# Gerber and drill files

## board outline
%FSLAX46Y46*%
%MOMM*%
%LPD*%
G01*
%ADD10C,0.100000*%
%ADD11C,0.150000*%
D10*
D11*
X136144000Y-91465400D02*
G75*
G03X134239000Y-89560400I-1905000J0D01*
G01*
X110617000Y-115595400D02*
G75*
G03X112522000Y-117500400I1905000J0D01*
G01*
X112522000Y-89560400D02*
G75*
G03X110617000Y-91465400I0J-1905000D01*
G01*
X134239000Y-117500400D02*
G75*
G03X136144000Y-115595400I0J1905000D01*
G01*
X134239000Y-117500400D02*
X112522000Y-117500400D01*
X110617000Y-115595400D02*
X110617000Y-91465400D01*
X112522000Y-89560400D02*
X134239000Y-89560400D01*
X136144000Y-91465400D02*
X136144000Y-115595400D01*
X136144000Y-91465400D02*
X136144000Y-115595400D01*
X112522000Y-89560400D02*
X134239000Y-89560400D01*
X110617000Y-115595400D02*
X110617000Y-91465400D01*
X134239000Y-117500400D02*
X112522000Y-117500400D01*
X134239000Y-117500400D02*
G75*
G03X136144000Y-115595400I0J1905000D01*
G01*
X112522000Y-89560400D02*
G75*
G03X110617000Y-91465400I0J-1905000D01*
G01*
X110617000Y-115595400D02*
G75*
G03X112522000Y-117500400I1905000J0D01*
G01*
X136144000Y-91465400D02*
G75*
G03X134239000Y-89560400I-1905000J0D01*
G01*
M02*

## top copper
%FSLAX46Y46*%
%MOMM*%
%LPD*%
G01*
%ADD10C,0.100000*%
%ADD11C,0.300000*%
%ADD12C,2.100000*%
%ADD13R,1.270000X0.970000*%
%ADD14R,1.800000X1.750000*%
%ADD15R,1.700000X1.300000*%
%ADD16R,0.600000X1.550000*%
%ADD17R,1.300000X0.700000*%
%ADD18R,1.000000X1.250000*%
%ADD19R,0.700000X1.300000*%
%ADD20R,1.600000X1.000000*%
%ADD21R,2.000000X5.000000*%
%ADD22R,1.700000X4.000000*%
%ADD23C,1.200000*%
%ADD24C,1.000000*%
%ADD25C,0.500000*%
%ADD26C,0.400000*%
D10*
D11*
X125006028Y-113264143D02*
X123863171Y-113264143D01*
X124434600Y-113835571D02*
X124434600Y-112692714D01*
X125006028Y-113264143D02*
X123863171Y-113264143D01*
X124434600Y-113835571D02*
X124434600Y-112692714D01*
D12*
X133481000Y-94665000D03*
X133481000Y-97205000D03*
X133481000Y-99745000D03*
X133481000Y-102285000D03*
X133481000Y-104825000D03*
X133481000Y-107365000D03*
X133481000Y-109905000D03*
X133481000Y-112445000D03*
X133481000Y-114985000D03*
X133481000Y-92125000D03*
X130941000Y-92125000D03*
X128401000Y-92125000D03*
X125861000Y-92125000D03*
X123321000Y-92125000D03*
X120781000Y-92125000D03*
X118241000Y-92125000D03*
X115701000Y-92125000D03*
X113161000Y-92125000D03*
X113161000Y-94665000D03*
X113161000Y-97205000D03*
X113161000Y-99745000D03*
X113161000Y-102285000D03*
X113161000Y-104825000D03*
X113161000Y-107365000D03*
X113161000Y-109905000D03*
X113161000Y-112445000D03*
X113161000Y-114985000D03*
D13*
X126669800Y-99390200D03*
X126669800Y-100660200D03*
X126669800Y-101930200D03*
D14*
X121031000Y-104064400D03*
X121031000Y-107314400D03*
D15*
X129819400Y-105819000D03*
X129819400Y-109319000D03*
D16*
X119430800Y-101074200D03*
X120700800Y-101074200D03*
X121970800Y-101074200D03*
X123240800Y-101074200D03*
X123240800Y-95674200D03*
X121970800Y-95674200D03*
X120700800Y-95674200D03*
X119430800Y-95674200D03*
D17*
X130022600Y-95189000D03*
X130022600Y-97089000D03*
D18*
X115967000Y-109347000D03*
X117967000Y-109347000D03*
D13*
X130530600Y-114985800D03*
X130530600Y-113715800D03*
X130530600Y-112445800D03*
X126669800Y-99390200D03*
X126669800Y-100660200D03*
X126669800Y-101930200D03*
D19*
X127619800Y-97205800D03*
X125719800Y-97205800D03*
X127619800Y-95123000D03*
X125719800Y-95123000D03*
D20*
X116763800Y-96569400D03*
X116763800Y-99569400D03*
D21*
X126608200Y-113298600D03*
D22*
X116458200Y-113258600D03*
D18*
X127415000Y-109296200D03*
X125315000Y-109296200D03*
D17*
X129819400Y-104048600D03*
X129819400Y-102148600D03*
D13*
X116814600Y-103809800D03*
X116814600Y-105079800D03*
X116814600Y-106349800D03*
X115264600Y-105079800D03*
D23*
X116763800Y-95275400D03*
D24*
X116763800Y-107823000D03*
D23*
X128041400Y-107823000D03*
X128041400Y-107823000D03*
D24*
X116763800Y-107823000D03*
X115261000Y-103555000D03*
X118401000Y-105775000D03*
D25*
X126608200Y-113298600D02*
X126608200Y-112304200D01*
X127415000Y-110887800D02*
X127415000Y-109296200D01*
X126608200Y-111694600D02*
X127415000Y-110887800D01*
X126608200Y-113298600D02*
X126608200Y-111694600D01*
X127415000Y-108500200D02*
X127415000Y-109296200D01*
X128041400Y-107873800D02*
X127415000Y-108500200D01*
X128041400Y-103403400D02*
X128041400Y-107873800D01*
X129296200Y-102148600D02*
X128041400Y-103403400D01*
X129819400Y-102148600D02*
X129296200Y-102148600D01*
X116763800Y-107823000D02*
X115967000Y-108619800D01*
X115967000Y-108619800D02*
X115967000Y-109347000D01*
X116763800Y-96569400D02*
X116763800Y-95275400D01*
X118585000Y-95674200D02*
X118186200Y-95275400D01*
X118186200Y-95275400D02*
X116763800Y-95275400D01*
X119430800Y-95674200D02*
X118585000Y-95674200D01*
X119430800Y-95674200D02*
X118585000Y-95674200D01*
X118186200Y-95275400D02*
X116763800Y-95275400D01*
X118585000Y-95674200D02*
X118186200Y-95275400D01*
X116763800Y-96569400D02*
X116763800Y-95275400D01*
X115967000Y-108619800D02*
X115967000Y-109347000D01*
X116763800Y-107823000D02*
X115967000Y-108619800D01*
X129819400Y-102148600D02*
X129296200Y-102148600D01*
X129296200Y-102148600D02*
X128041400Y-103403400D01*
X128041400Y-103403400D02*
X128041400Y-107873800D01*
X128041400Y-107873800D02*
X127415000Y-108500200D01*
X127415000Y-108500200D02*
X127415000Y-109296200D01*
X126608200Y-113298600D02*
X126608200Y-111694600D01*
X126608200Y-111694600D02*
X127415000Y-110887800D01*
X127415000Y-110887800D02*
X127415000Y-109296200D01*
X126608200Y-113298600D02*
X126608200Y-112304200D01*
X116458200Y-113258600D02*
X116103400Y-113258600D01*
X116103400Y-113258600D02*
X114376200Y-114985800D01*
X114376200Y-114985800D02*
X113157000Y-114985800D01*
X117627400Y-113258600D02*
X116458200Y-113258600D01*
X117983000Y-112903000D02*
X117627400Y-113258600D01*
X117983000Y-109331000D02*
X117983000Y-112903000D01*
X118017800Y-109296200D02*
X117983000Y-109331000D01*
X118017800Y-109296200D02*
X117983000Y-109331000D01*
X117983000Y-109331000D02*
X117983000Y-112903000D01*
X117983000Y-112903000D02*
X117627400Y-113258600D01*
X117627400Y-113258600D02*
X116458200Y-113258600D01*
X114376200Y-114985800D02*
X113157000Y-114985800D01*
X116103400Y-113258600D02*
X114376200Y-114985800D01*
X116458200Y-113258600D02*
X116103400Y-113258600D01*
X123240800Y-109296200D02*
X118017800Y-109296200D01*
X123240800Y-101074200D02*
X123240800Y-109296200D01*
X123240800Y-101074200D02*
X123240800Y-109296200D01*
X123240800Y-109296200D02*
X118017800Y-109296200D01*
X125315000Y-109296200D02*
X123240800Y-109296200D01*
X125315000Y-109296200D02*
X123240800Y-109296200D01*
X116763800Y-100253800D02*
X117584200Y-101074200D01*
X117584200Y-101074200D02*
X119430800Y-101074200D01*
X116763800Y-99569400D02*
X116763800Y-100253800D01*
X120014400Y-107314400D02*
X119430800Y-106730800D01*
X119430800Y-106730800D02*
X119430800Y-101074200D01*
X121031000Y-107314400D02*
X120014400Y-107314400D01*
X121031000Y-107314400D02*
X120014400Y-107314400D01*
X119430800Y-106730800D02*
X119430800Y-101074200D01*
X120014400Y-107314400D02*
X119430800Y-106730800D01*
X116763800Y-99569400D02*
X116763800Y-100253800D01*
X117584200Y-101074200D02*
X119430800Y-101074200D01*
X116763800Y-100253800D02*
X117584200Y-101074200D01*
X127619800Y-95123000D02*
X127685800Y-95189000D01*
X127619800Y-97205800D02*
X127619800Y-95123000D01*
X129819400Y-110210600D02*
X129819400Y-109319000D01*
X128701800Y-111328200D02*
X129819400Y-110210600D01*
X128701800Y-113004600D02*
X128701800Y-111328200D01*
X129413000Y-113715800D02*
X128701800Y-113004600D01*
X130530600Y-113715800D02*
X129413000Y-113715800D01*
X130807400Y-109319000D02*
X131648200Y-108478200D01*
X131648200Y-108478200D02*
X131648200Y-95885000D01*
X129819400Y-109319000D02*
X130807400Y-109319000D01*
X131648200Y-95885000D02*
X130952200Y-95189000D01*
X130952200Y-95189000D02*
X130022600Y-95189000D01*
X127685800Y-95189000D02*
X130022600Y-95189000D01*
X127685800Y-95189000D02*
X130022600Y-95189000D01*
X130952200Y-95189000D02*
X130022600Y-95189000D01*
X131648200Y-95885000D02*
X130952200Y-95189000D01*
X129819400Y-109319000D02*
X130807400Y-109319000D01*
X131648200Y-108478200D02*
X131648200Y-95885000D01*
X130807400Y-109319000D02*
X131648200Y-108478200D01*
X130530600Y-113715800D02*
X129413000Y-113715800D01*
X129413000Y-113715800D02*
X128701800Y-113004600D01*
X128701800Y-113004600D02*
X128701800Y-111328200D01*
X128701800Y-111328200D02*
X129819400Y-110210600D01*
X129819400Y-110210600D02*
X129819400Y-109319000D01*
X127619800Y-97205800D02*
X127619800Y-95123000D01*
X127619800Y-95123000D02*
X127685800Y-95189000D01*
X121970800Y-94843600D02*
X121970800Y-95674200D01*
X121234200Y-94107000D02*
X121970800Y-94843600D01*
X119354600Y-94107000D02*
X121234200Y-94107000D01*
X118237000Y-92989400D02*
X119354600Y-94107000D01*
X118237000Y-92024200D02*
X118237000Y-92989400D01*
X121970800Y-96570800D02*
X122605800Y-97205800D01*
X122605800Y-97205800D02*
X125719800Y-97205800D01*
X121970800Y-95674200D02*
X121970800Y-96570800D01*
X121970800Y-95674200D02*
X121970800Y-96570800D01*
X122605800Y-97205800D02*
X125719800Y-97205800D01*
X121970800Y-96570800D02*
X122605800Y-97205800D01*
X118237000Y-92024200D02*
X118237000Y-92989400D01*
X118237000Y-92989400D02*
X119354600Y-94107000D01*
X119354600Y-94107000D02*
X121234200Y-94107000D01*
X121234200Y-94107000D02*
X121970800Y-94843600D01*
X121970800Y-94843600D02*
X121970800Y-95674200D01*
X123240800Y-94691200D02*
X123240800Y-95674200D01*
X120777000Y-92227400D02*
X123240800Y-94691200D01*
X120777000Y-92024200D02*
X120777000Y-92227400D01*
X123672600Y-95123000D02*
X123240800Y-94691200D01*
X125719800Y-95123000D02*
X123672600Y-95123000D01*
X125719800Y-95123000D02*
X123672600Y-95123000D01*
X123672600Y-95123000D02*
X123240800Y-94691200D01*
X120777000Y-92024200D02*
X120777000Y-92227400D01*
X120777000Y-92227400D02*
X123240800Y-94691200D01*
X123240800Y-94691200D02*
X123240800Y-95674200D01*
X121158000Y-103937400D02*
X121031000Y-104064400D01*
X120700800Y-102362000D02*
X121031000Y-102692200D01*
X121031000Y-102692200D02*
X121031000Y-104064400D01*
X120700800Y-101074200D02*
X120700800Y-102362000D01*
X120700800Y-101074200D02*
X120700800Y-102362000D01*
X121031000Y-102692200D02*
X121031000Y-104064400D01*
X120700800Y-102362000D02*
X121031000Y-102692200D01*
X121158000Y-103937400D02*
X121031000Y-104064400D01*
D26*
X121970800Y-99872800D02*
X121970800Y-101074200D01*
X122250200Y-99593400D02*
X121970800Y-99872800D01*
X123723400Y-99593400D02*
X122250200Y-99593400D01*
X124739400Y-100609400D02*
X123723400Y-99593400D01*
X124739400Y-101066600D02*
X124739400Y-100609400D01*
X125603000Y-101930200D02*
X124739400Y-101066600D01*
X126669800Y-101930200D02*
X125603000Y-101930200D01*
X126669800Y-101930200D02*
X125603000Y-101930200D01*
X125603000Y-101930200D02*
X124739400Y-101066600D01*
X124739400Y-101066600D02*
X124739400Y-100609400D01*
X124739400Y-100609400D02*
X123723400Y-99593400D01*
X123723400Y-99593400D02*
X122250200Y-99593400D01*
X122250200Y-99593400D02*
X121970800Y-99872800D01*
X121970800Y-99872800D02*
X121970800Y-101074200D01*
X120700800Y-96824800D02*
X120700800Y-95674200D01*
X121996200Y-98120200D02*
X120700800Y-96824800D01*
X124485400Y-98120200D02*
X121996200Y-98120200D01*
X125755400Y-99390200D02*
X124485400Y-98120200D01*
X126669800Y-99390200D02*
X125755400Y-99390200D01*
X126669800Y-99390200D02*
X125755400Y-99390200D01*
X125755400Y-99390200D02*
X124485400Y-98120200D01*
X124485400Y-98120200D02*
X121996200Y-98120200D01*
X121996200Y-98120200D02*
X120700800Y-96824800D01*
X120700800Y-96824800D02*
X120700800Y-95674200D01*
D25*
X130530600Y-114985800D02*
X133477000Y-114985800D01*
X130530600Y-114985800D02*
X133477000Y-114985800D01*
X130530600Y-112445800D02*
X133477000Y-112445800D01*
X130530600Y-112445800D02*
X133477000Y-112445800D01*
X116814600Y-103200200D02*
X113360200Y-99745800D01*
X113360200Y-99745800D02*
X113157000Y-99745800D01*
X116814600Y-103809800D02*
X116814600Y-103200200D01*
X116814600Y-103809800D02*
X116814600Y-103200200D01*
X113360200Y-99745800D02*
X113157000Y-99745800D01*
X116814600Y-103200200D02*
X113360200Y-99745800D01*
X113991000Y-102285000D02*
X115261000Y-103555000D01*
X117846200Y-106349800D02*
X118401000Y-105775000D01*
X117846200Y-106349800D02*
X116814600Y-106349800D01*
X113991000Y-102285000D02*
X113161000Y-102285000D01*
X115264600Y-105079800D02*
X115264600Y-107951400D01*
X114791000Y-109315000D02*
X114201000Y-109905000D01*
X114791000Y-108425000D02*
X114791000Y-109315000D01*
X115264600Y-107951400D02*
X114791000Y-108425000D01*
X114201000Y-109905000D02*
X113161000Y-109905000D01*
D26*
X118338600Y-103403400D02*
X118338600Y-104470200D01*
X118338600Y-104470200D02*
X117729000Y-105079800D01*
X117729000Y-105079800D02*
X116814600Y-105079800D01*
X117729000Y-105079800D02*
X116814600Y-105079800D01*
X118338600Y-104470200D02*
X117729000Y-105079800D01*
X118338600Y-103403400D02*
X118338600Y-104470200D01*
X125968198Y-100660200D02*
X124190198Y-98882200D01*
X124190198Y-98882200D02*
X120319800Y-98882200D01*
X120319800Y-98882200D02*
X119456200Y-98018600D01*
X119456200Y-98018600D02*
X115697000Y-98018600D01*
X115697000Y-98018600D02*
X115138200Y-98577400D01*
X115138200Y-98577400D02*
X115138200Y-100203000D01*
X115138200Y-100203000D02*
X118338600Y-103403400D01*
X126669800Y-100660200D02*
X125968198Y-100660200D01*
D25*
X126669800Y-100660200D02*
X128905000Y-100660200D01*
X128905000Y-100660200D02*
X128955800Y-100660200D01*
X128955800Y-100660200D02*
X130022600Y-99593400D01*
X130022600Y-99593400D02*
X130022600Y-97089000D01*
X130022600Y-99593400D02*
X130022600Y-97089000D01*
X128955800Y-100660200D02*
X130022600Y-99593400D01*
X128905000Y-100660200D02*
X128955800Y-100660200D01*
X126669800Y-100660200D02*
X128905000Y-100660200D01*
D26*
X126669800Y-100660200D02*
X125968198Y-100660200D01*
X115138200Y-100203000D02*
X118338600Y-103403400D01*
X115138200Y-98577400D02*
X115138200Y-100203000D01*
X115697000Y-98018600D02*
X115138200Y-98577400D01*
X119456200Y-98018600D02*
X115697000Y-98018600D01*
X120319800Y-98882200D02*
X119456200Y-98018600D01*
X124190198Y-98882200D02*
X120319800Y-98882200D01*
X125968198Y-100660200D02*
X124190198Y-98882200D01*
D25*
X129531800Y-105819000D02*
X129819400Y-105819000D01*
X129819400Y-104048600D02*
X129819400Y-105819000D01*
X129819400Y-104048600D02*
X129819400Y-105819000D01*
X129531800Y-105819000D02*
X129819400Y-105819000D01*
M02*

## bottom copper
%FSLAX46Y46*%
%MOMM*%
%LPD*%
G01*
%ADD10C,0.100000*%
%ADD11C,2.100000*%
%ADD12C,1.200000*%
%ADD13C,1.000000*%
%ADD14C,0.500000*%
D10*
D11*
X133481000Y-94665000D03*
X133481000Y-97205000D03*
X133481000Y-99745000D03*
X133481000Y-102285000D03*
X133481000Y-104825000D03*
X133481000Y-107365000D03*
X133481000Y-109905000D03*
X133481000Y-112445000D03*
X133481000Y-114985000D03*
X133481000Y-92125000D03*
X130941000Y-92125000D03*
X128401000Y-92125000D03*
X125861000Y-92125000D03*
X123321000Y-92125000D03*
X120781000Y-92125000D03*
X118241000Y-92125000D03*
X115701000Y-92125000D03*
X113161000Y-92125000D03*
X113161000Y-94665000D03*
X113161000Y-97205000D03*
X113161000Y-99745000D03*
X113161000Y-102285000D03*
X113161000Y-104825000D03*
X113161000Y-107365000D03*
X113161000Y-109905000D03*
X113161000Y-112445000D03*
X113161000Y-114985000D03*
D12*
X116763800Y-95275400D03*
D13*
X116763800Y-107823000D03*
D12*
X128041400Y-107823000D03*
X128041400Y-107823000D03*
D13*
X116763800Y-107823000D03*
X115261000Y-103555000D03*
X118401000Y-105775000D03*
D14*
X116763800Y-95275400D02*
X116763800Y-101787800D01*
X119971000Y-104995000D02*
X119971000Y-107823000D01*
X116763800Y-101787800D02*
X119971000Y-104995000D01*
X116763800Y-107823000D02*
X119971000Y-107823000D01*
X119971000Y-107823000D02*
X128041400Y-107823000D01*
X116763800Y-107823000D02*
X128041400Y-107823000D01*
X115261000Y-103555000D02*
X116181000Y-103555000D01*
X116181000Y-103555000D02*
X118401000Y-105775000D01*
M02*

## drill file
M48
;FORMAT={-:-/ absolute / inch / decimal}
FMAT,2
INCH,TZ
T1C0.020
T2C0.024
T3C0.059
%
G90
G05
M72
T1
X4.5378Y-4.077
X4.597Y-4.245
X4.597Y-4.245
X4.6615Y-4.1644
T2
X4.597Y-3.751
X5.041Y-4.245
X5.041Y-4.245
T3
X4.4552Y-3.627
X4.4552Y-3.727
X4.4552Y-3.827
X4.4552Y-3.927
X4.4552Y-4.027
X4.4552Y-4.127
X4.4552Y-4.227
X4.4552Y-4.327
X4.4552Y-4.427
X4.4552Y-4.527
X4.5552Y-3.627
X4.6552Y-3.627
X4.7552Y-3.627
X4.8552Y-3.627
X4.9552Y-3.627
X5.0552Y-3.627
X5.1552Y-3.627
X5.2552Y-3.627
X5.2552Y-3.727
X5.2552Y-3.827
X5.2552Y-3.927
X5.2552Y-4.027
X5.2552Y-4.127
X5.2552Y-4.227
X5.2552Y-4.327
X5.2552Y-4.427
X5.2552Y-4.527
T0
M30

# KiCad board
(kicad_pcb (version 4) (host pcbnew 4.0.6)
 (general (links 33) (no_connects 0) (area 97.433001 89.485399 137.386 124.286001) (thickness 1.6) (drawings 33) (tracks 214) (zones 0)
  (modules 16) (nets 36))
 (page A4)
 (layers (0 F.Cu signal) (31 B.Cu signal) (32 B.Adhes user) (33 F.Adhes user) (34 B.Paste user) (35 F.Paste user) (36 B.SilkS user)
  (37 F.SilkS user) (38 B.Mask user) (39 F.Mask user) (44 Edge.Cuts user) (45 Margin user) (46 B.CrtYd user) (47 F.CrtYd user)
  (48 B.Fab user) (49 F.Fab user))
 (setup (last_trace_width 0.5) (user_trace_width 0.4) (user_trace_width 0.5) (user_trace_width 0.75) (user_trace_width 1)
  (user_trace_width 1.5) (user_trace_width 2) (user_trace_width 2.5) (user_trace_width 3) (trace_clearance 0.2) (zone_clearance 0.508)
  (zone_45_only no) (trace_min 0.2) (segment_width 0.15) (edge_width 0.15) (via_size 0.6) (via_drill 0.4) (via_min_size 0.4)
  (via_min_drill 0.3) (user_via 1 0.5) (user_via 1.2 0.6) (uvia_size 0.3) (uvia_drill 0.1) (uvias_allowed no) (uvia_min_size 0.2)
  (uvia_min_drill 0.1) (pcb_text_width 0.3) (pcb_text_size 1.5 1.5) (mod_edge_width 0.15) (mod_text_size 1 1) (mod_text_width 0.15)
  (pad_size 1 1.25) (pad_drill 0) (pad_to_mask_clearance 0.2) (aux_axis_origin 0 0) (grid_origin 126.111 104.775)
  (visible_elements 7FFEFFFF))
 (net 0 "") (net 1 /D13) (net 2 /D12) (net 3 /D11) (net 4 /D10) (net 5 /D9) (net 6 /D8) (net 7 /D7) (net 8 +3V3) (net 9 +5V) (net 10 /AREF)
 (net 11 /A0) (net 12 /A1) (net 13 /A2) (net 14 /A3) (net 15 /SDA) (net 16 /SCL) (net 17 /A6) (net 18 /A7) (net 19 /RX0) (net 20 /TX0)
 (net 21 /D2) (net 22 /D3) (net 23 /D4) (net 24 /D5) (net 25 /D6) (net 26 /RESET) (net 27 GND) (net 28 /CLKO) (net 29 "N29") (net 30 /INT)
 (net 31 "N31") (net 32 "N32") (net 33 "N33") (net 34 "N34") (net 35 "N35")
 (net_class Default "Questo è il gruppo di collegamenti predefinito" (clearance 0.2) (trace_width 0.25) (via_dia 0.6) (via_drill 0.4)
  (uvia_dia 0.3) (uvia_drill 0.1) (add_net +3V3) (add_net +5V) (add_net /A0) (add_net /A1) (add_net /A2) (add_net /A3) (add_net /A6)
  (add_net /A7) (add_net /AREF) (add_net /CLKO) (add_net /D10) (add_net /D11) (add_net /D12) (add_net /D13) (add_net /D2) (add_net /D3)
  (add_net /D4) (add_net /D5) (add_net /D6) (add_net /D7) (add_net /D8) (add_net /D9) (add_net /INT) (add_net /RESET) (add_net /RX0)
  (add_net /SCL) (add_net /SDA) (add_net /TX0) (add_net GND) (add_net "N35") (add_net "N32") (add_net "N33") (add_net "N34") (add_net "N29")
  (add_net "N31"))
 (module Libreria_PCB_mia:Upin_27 (layer B.Cu) (at 133.481 114.985 180)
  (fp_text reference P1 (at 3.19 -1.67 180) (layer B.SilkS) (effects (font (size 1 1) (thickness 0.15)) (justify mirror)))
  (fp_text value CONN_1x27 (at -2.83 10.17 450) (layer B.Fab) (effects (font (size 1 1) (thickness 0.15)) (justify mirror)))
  (pad 9 thru_hole circle (at 0 20.32 180) (size 2.1 2.1) (drill 1.5) (layers *.Cu *.Mask) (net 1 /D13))
  (pad 8 thru_hole circle (at 0 17.78 180) (size 2.1 2.1) (drill 1.5) (layers *.Cu *.Mask) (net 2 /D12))
  (pad 7 thru_hole circle (at 0 15.24 180) (size 2.1 2.1) (drill 1.5) (layers *.Cu *.Mask) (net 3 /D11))
  (pad 6 thru_hole circle (at 0 12.7 180) (size 2.1 2.1) (drill 1.5) (layers *.Cu *.Mask) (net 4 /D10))
  (pad 5 thru_hole circle (at 0 10.16 180) (size 2.1 2.1) (drill 1.5) (layers *.Cu *.Mask) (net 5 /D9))
  (pad 4 thru_hole circle (at 0 7.62 180) (size 2.1 2.1) (drill 1.5) (layers *.Cu *.Mask) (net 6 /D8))
  (pad 3 thru_hole circle (at 0 5.08 180) (size 2.1 2.1) (drill 1.5) (layers *.Cu *.Mask) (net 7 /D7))
  (pad 2 thru_hole circle (at 0 2.54 180) (size 2.1 2.1) (drill 1.5) (layers *.Cu *.Mask) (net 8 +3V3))
  (pad 1 thru_hole circle (at 0 0 180) (size 2.1 2.1) (drill 1.5) (layers *.Cu *.Mask) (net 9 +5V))
  (pad 10 thru_hole circle (at 0 22.86 180) (size 2.1 2.1) (drill 1.5) (layers *.Cu *.Mask) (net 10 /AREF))
  (pad 11 thru_hole circle (at 2.54 22.86 180) (size 2.1 2.1) (drill 1.5) (layers *.Cu *.Mask) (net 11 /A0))
  (pad 12 thru_hole circle (at 5.08 22.86 180) (size 2.1 2.1) (drill 1.5) (layers *.Cu *.Mask) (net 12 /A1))
  (pad 13 thru_hole circle (at 7.62 22.86 180) (size 2.1 2.1) (drill 1.5) (layers *.Cu *.Mask) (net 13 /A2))
  (pad 14 thru_hole circle (at 10.16 22.86 180) (size 2.1 2.1) (drill 1.5) (layers *.Cu *.Mask) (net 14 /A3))
  (pad 15 thru_hole circle (at 12.7 22.86 180) (size 2.1 2.1) (drill 1.5) (layers *.Cu *.Mask) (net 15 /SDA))
  (pad 16 thru_hole circle (at 15.24 22.86 180) (size 2.1 2.1) (drill 1.5) (layers *.Cu *.Mask) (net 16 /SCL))
  (pad 17 thru_hole circle (at 17.78 22.86 180) (size 2.1 2.1) (drill 1.5) (layers *.Cu *.Mask) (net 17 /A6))
  (pad 18 thru_hole circle (at 20.32 22.86 180) (size 2.1 2.1) (drill 1.5) (layers *.Cu *.Mask) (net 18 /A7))
  (pad 19 thru_hole circle (at 20.32 20.32 180) (size 2.1 2.1) (drill 1.5) (layers *.Cu *.Mask) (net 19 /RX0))
  (pad 20 thru_hole circle (at 20.32 17.78 180) (size 2.1 2.1) (drill 1.5) (layers *.Cu *.Mask) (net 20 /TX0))
  (pad 21 thru_hole circle (at 20.32 15.24 180) (size 2.1 2.1) (drill 1.5) (layers *.Cu *.Mask) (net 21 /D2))
  (pad 22 thru_hole circle (at 20.32 12.7 180) (size 2.1 2.1) (drill 1.5) (layers *.Cu *.Mask) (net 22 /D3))
  (pad 23 thru_hole circle (at 20.32 10.16 180) (size 2.1 2.1) (drill 1.5) (layers *.Cu *.Mask) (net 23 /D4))
  (pad 24 thru_hole circle (at 20.32 7.62 180) (size 2.1 2.1) (drill 1.5) (layers *.Cu *.Mask) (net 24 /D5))
  (pad 25 thru_hole circle (at 20.32 5.08 180) (size 2.1 2.1) (drill 1.5) (layers *.Cu *.Mask) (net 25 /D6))
  (pad 26 thru_hole circle (at 20.32 2.54 180) (size 2.1 2.1) (drill 1.5) (layers *.Cu *.Mask) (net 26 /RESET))
  (pad 27 thru_hole circle (at 20.32 0 180) (size 2.1 2.1) (drill 1.5) (layers *.Cu *.Mask) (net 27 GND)))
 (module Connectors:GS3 (layer F.Cu) (at 126.6698 100.6602)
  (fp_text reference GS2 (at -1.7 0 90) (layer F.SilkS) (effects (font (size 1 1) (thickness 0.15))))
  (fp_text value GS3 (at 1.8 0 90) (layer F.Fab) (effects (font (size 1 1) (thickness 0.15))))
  (pad 1 smd rect (at 0 -1.27) (size 1.27 0.97) (layers F.Cu F.Paste F.Mask) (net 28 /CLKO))
  (pad 2 smd rect (at 0 0) (size 1.27 0.97) (layers F.Cu F.Paste F.Mask) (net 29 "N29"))
  (pad 3 smd rect (at 0 1.27) (size 1.27 0.97) (layers F.Cu F.Paste F.Mask) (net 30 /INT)))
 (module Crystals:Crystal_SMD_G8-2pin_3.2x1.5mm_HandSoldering (layer F.Cu) (at 121.031 105.6894 270)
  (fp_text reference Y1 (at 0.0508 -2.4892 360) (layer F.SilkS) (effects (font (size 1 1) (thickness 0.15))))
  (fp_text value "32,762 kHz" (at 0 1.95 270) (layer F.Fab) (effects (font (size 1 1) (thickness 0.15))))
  (pad 1 smd rect (at -1.625 0 270) (size 1.75 1.8) (layers F.Cu F.Paste F.Mask) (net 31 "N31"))
  (pad 2 smd rect (at 1.625 0 270) (size 1.75 1.8) (layers F.Cu F.Paste F.Mask) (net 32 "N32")))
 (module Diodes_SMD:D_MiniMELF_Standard (layer F.Cu) (at 129.8194 107.569 270)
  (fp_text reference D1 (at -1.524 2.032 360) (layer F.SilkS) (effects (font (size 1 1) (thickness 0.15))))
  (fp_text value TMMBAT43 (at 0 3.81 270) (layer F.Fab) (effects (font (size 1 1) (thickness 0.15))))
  (pad 1 smd rect (at -1.75 0 270) (size 1.3 1.7) (layers F.Cu F.Paste F.Mask) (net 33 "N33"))
  (pad 2 smd rect (at 1.75 0 270) (size 1.3 1.7) (layers F.Cu F.Paste F.Mask) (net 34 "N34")))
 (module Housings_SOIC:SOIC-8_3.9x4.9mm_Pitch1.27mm (layer F.Cu) (at 121.3358 98.3742 90)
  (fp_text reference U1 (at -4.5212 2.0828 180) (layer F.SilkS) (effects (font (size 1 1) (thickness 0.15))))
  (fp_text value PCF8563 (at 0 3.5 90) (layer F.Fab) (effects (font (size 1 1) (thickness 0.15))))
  (pad 1 smd rect (at -2.7 -1.905 90) (size 1.55 0.6) (layers F.Cu F.Paste F.Mask) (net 32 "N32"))
  (pad 2 smd rect (at -2.7 -0.635 90) (size 1.55 0.6) (layers F.Cu F.Paste F.Mask) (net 31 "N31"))
  (pad 3 smd rect (at -2.7 0.635 90) (size 1.55 0.6) (layers F.Cu F.Paste F.Mask) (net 30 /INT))
  (pad 4 smd rect (at -2.7 1.905 90) (size 1.55 0.6) (layers F.Cu F.Paste F.Mask) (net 27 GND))
  (pad 5 smd rect (at 2.7 1.905 90) (size 1.55 0.6) (layers F.Cu F.Paste F.Mask) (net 15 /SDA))
  (pad 6 smd rect (at 2.7 0.635 90) (size 1.55 0.6) (layers F.Cu F.Paste F.Mask) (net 16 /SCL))
  (pad 7 smd rect (at 2.7 -0.635 90) (size 1.55 0.6) (layers F.Cu F.Paste F.Mask) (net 28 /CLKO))
  (pad 8 smd rect (at 2.7 -1.905 90) (size 1.55 0.6) (layers F.Cu F.Paste F.Mask) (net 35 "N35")))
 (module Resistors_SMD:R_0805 (layer F.Cu) (at 130.0226 96.139 270)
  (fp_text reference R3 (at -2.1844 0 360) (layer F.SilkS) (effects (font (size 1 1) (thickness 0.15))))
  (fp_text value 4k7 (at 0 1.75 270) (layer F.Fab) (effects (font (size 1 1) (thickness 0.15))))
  (pad 1 smd rect (at -0.95 0 270) (size 0.7 1.3) (layers F.Cu F.Paste F.Mask) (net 34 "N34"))
  (pad 2 smd rect (at 0.95 0 270) (size 0.7 1.3) (layers F.Cu F.Paste F.Mask) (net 29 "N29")))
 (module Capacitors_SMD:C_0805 (layer F.Cu) (at 116.967 109.347)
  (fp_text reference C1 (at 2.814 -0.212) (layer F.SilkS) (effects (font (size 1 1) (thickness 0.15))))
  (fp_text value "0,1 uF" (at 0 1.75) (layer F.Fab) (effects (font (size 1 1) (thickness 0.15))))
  (pad 1 smd rect (at -1 0) (size 1 1.25) (layers F.Cu F.Paste F.Mask) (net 35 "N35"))
  (pad 2 smd rect (at 1 0) (size 1 1.25) (layers F.Cu F.Paste F.Mask) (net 27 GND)))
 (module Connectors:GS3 (layer F.Cu) (at 130.5306 113.7158 180)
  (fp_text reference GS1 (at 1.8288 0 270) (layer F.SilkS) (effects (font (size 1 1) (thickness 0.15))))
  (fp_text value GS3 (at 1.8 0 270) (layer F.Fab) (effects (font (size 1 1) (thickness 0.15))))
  (pad 1 smd rect (at 0 -1.27 180) (size 1.27 0.97) (layers F.Cu F.Paste F.Mask) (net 9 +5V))
  (pad 2 smd rect (at 0 0 180) (size 1.27 0.97) (layers F.Cu F.Paste F.Mask) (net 34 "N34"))
  (pad 3 smd rect (at 0 1.27 180) (size 1.27 0.97) (layers F.Cu F.Paste F.Mask) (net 8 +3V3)))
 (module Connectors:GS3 (layer F.Cu) (at 126.6698 100.6602)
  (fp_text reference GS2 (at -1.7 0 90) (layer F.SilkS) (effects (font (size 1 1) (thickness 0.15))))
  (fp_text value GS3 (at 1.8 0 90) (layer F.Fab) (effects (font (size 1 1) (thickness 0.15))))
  (pad 1 smd rect (at 0 -1.27) (size 1.27 0.97) (layers F.Cu F.Paste F.Mask) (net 28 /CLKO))
  (pad 2 smd rect (at 0 0) (size 1.27 0.97) (layers F.Cu F.Paste F.Mask) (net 29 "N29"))
  (pad 3 smd rect (at 0 1.27) (size 1.27 0.97) (layers F.Cu F.Paste F.Mask) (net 30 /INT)))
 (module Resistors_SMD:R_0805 (layer F.Cu) (at 126.6698 97.2058 180)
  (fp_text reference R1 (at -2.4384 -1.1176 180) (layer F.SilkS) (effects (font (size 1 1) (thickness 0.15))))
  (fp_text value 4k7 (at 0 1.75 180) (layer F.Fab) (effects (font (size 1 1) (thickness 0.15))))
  (pad 1 smd rect (at -0.95 0 180) (size 0.7 1.3) (layers F.Cu F.Paste F.Mask) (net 34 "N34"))
  (pad 2 smd rect (at 0.95 0 180) (size 0.7 1.3) (layers F.Cu F.Paste F.Mask) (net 16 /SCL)))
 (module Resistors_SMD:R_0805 (layer F.Cu) (at 126.6698 95.123 180)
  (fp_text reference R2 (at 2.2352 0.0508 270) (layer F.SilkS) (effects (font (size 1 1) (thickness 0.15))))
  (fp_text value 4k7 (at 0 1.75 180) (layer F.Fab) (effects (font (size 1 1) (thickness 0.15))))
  (pad 1 smd rect (at -0.95 0 180) (size 0.7 1.3) (layers F.Cu F.Paste F.Mask) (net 34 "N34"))
  (pad 2 smd rect (at 0.95 0 180) (size 0.7 1.3) (layers F.Cu F.Paste F.Mask) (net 15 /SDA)))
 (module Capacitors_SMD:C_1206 (layer F.Cu) (at 116.7638 98.0694 270)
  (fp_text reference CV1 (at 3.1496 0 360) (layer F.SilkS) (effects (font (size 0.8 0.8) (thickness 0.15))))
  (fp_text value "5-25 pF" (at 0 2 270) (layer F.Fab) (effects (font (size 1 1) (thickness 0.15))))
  (pad 1 smd rect (at -1.5 0 270) (size 1 1.6) (layers F.Cu F.Paste F.Mask) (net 35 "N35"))
  (pad 2 smd rect (at 1.5 0 270) (size 1 1.6) (layers F.Cu F.Paste F.Mask) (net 32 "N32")))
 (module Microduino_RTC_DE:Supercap (layer F.Cu) (at 121.4882 113.2586 180)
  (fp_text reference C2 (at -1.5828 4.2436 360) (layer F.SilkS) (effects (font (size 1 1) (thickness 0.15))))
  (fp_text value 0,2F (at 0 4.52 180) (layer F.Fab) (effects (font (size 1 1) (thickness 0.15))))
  (pad 1 smd rect (at -5.12 -0.04 180) (size 2 5) (layers F.Cu F.Paste F.Mask) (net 35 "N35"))
  (pad 2 smd rect (at 5.03 0 180) (size 1.7 4) (layers F.Cu F.Mask) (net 27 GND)))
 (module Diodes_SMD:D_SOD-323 (layer F.Cu) (at 126.365 109.2962 180)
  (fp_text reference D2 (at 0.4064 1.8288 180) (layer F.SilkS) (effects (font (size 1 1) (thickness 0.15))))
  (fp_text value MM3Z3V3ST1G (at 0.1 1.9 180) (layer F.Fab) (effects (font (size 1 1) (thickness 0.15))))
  (pad 1 smd rect (at -1.05 0 180) (size 1 1.25) (layers F.Cu F.Paste F.Mask) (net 35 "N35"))
  (pad 2 smd rect (at 1.05 0 180) (size 1 1.25) (layers F.Cu F.Paste F.Mask) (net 27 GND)))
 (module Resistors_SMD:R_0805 (layer F.Cu) (at 129.8194 103.0986 90)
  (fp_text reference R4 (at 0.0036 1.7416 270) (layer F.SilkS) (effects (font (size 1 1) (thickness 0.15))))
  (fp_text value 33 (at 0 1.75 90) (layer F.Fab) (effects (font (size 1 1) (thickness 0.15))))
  (pad 1 smd rect (at -0.95 0 90) (size 0.7 1.3) (layers F.Cu F.Paste F.Mask) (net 33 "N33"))
  (pad 2 smd rect (at 0.95 0 90) (size 0.7 1.3) (layers F.Cu F.Paste F.Mask) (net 35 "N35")))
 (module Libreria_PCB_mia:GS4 (layer F.Cu) (at 116.8146 105.0798)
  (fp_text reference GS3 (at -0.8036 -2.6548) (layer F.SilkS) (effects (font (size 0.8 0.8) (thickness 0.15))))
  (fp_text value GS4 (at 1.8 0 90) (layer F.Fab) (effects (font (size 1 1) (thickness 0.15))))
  (pad 1 smd rect (at 0 -1.27) (size 1.27 0.97) (layers F.Cu F.Paste F.Mask) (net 21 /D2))
  (pad 2 smd rect (at 0 0) (size 1.27 0.97) (layers F.Cu F.Paste F.Mask) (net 29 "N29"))
  (pad 3 smd rect (at 0 1.27) (size 1.27 0.97) (layers F.Cu F.Paste F.Mask) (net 22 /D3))
  (pad 4 smd rect (at -1.55 0) (size 1.27 0.97) (layers F.Cu F.Paste F.Mask) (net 25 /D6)))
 (gr_arc (start 134.239 91.4654) (end 134.239 89.5604) (angle 90) (layer Edge.Cuts) (width 0.15))
 (gr_arc (start 112.522 115.5954) (end 112.522 117.5004) (angle 90) (layer Edge.Cuts) (width 0.15))
 (gr_arc (start 112.522 91.4654) (end 110.617 91.4654) (angle 90) (layer Edge.Cuts) (width 0.15))
 (gr_arc (start 134.239 115.5954) (end 136.144 115.5954) (angle 90) (layer Edge.Cuts) (width 0.15))
 (gr_line (start 134.239 117.5004) (end 112.522 117.5004) (angle 90) (layer Edge.Cuts) (width 0.15))
 (gr_line (start 110.617 115.5954) (end 110.617 91.4654) (angle 90) (layer Edge.Cuts) (width 0.15))
 (gr_line (start 112.522 89.5604) (end 134.239 89.5604) (angle 90) (layer Edge.Cuts) (width 0.15))
 (gr_line (start 136.144 91.4654) (end 136.144 115.5954) (angle 90) (layer Edge.Cuts) (width 0.15))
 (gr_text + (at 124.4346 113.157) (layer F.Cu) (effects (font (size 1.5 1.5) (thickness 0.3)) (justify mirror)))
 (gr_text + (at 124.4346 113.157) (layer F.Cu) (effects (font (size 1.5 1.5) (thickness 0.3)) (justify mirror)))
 (gr_line (start 136.144 91.4654) (end 136.144 115.5954) (angle 90) (layer Edge.Cuts) (width 0.15))
 (gr_line (start 112.522 89.5604) (end 134.239 89.5604) (angle 90) (layer Edge.Cuts) (width 0.15))
 (gr_line (start 110.617 115.5954) (end 110.617 91.4654) (angle 90) (layer Edge.Cuts) (width 0.15))
 (gr_line (start 134.239 117.5004) (end 112.522 117.5004) (angle 90) (layer Edge.Cuts) (width 0.15))
 (gr_arc (start 134.239 115.5954) (end 136.144 115.5954) (angle 90) (layer Edge.Cuts) (width 0.15))
 (gr_arc (start 112.522 91.4654) (end 110.617 91.4654) (angle 90) (layer Edge.Cuts) (width 0.15))
 (gr_arc (start 112.522 115.5954) (end 112.522 117.5004) (angle 90) (layer Edge.Cuts) (width 0.15))
 (gr_arc (start 134.239 91.4654) (end 134.239 89.5604) (angle 90) (layer Edge.Cuts) (width 0.15))
 (segment (start 116.7638 95.2754) (end 116.7638 101.7878) (width 0.5) (layer B.Cu) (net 35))
 (via (at 116.7638 95.2754) (size 1.2) (drill 0.6) (layers F.Cu B.Cu) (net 35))
 (segment (start 119.971 104.995) (end 119.971 107.823) (width 0.5) (layer B.Cu) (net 35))
 (segment (start 116.7638 101.7878) (end 119.971 104.995) (width 0.5) (layer B.Cu) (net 35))
 (segment (start 126.6082 113.2986) (end 126.6082 112.3042) (width 0.5) (layer F.Cu) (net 35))
 (segment (start 127.415 110.8878) (end 127.415 109.2962) (width 0.5) (layer F.Cu) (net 35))
 (segment (start 126.6082 111.6946) (end 127.415 110.8878) (width 0.5) (layer F.Cu) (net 35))
 (segment (start 126.6082 113.2986) (end 126.6082 111.6946) (width 0.5) (layer F.Cu) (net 35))
 (segment (start 127.415 108.5002) (end 127.415 109.2962) (width 0.5) (layer F.Cu) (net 35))
 (segment (start 128.0414 107.8738) (end 127.415 108.5002) (width 0.5) (layer F.Cu) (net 35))
 (segment (start 128.0414 103.4034) (end 128.0414 107.8738) (width 0.5) (layer F.Cu) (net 35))
 (segment (start 129.2962 102.1486) (end 128.0414 103.4034) (width 0.5) (layer F.Cu) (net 35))
 (segment (start 129.8194 102.1486) (end 129.2962 102.1486) (width 0.5) (layer F.Cu) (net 35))
 (via (at 116.7638 107.823) (size 1) (drill 0.5) (layers F.Cu B.Cu) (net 35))
 (segment (start 116.7638 107.823) (end 115.967 108.6198) (width 0.5) (layer F.Cu) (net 35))
 (segment (start 115.967 108.6198) (end 115.967 109.347) (width 0.5) (layer F.Cu) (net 35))
 (segment (start 116.7638 96.5694) (end 116.7638 95.2754) (width 0.5) (layer F.Cu) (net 35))
 (segment (start 118.585 95.6742) (end 118.1862 95.2754) (width 0.5) (layer F.Cu) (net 35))
 (segment (start 118.1862 95.2754) (end 116.7638 95.2754) (width 0.5) (layer F.Cu) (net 35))
 (segment (start 119.4308 95.6742) (end 118.585 95.6742) (width 0.5) (layer F.Cu) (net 35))
 (via (at 128.0414 107.823) (size 1.2) (drill 0.6) (layers F.Cu B.Cu) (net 35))
 (segment (start 116.7638 107.823) (end 119.971 107.823) (width 0.5) (layer B.Cu) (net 35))
 (segment (start 119.971 107.823) (end 128.0414 107.823) (width 0.5) (layer B.Cu) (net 35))
 (segment (start 116.7638 107.823) (end 128.0414 107.823) (width 0.5) (layer B.Cu) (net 35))
 (via (at 128.0414 107.823) (size 1.2) (drill 0.6) (layers F.Cu B.Cu) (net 35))
 (segment (start 119.4308 95.6742) (end 118.585 95.6742) (width 0.5) (layer F.Cu) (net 35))
 (segment (start 118.1862 95.2754) (end 116.7638 95.2754) (width 0.5) (layer F.Cu) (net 35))
 (segment (start 118.585 95.6742) (end 118.1862 95.2754) (width 0.5) (layer F.Cu) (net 35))
 (segment (start 116.7638 96.5694) (end 116.7638 95.2754) (width 0.5) (layer F.Cu) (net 35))
 (segment (start 115.967 108.6198) (end 115.967 109.347) (width 0.5) (layer F.Cu) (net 35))
 (segment (start 116.7638 107.823) (end 115.967 108.6198) (width 0.5) (layer F.Cu) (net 35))
 (via (at 116.7638 107.823) (size 1) (drill 0.5) (layers F.Cu B.Cu) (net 35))
 (segment (start 129.8194 102.1486) (end 129.2962 102.1486) (width 0.5) (layer F.Cu) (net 35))
 (segment (start 129.2962 102.1486) (end 128.0414 103.4034) (width 0.5) (layer F.Cu) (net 35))
 (segment (start 128.0414 103.4034) (end 128.0414 107.8738) (width 0.5) (layer F.Cu) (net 35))
 (segment (start 128.0414 107.8738) (end 127.415 108.5002) (width 0.5) (layer F.Cu) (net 35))
 (segment (start 127.415 108.5002) (end 127.415 109.2962) (width 0.5) (layer F.Cu) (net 35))
 (segment (start 126.6082 113.2986) (end 126.6082 111.6946) (width 0.5) (layer F.Cu) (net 35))
 (segment (start 126.6082 111.6946) (end 127.415 110.8878) (width 0.5) (layer F.Cu) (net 35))
 (segment (start 127.415 110.8878) (end 127.415 109.2962) (width 0.5) (layer F.Cu) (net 35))
 (segment (start 126.6082 113.2986) (end 126.6082 112.3042) (width 0.5) (layer F.Cu) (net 35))
 (segment (start 116.4582 113.2586) (end 116.1034 113.2586) (width 0.5) (layer F.Cu) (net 27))
 (segment (start 116.1034 113.2586) (end 114.3762 114.9858) (width 0.5) (layer F.Cu) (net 27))
 (segment (start 114.3762 114.9858) (end 113.157 114.9858) (width 0.5) (layer F.Cu) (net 27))
 (segment (start 117.6274 113.2586) (end 116.4582 113.2586) (width 0.5) (layer F.Cu) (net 27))
 (segment (start 117.983 112.903) (end 117.6274 113.2586) (width 0.5) (layer F.Cu) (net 27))
 (segment (start 117.983 109.331) (end 117.983 112.903) (width 0.5) (layer F.Cu) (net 27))
 (segment (start 118.0178 109.2962) (end 117.983 109.331) (width 0.5) (layer F.Cu) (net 27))
 (segment (start 118.0178 109.2962) (end 117.983 109.331) (width 0.5) (layer F.Cu) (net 27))
 (segment (start 117.983 109.331) (end 117.983 112.903) (width 0.5) (layer F.Cu) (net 27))
 (segment (start 117.983 112.903) (end 117.6274 113.2586) (width 0.5) (layer F.Cu) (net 27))
 (segment (start 117.6274 113.2586) (end 116.4582 113.2586) (width 0.5) (layer F.Cu) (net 27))
 (segment (start 114.3762 114.9858) (end 113.157 114.9858) (width 0.5) (layer F.Cu) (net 27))
 (segment (start 116.1034 113.2586) (end 114.3762 114.9858) (width 0.5) (layer F.Cu) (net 27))
 (segment (start 116.4582 113.2586) (end 116.1034 113.2586) (width 0.5) (layer F.Cu) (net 27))
 (segment (start 123.2408 109.2962) (end 118.0178 109.2962) (width 0.5) (layer F.Cu) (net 27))
 (segment (start 123.2408 101.0742) (end 123.2408 109.2962) (width 0.5) (layer F.Cu) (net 27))
 (segment (start 123.2408 101.0742) (end 123.2408 109.2962) (width 0.5) (layer F.Cu) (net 27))
 (segment (start 123.2408 109.2962) (end 118.0178 109.2962) (width 0.5) (layer F.Cu) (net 27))
 (segment (start 125.315 109.2962) (end 123.2408 109.2962) (width 0.5) (layer F.Cu) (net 27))
 (segment (start 125.315 109.2962) (end 123.2408 109.2962) (width 0.5) (layer F.Cu) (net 27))
 (segment (start 116.7638 100.2538) (end 117.5842 101.0742) (width 0.5) (layer F.Cu) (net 32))
 (segment (start 117.5842 101.0742) (end 119.4308 101.0742) (width 0.5) (layer F.Cu) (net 32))
 (segment (start 116.7638 99.5694) (end 116.7638 100.2538) (width 0.5) (layer F.Cu) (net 32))
 (segment (start 120.0144 107.3144) (end 119.4308 106.7308) (width 0.5) (layer F.Cu) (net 32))
 (segment (start 119.4308 106.7308) (end 119.4308 101.0742) (width 0.5) (layer F.Cu) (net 32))
 (segment (start 121.031 107.3144) (end 120.0144 107.3144) (width 0.5) (layer F.Cu) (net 32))
 (segment (start 121.031 107.3144) (end 120.0144 107.3144) (width 0.5) (layer F.Cu) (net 32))
 (segment (start 119.4308 106.7308) (end 119.4308 101.0742) (width 0.5) (layer F.Cu) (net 32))
 (segment (start 120.0144 107.3144) (end 119.4308 106.7308) (width 0.5) (layer F.Cu) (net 32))
 (segment (start 116.7638 99.5694) (end 116.7638 100.2538) (width 0.5) (layer F.Cu) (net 32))
 (segment (start 117.5842 101.0742) (end 119.4308 101.0742) (width 0.5) (layer F.Cu) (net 32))
 (segment (start 116.7638 100.2538) (end 117.5842 101.0742) (width 0.5) (layer F.Cu) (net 32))
 (segment (start 127.6198 95.123) (end 127.6858 95.189) (width 0.5) (layer F.Cu) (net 34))
 (segment (start 127.6198 97.2058) (end 127.6198 95.123) (width 0.5) (layer F.Cu) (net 34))
 (segment (start 129.8194 110.2106) (end 129.8194 109.319) (width 0.5) (layer F.Cu) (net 34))
 (segment (start 128.7018 111.3282) (end 129.8194 110.2106) (width 0.5) (layer F.Cu) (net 34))
 (segment (start 128.7018 113.0046) (end 128.7018 111.3282) (width 0.5) (layer F.Cu) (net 34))
 (segment (start 129.413 113.7158) (end 128.7018 113.0046) (width 0.5) (layer F.Cu) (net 34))
 (segment (start 130.5306 113.7158) (end 129.413 113.7158) (width 0.5) (layer F.Cu) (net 34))
 (segment (start 130.8074 109.319) (end 131.6482 108.4782) (width 0.5) (layer F.Cu) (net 34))
 (segment (start 131.6482 108.4782) (end 131.6482 95.885) (width 0.5) (layer F.Cu) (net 34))
 (segment (start 129.8194 109.319) (end 130.8074 109.319) (width 0.5) (layer F.Cu) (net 34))
 (segment (start 131.6482 95.885) (end 130.9522 95.189) (width 0.5) (layer F.Cu) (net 34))
 (segment (start 130.9522 95.189) (end 130.0226 95.189) (width 0.5) (layer F.Cu) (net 34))
 (segment (start 127.6858 95.189) (end 130.0226 95.189) (width 0.5) (layer F.Cu) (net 34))
 (segment (start 127.6858 95.189) (end 130.0226 95.189) (width 0.5) (layer F.Cu) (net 34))
 (segment (start 130.9522 95.189) (end 130.0226 95.189) (width 0.5) (layer F.Cu) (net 34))
 (segment (start 131.6482 95.885) (end 130.9522 95.189) (width 0.5) (layer F.Cu) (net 34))
 (segment (start 129.8194 109.319) (end 130.8074 109.319) (width 0.5) (layer F.Cu) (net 34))
 (segment (start 131.6482 108.4782) (end 131.6482 95.885) (width 0.5) (layer F.Cu) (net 34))
 (segment (start 130.8074 109.319) (end 131.6482 108.4782) (width 0.5) (layer F.Cu) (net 34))
 (segment (start 130.5306 113.7158) (end 129.413 113.7158) (width 0.5) (layer F.Cu) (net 34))
 (segment (start 129.413 113.7158) (end 128.7018 113.0046) (width 0.5) (layer F.Cu) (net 34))
 (segment (start 128.7018 113.0046) (end 128.7018 111.3282) (width 0.5) (layer F.Cu) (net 34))
 (segment (start 128.7018 111.3282) (end 129.8194 110.2106) (width 0.5) (layer F.Cu) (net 34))
 (segment (start 129.8194 110.2106) (end 129.8194 109.319) (width 0.5) (layer F.Cu) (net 34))
 (segment (start 127.6198 97.2058) (end 127.6198 95.123) (width 0.5) (layer F.Cu) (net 34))
 (segment (start 127.6198 95.123) (end 127.6858 95.189) (width 0.5) (layer F.Cu) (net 34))
 (segment (start 121.9708 94.8436) (end 121.9708 95.6742) (width 0.5) (layer F.Cu) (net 16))
 (segment (start 121.2342 94.107) (end 121.9708 94.8436) (width 0.5) (layer F.Cu) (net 16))
 (segment (start 119.3546 94.107) (end 121.2342 94.107) (width 0.5) (layer F.Cu) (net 16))
 (segment (start 118.237 92.9894) (end 119.3546 94.107) (width 0.5) (layer F.Cu) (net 16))
 (segment (start 118.237 92.0242) (end 118.237 92.9894) (width 0.5) (layer F.Cu) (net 16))
 (segment (start 121.9708 96.5708) (end 122.6058 97.2058) (width 0.5) (layer F.Cu) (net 16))
 (segment (start 122.6058 97.2058) (end 125.7198 97.2058) (width 0.5) (layer F.Cu) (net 16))
 (segment (start 121.9708 95.6742) (end 121.9708 96.5708) (width 0.5) (layer F.Cu) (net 16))
 (segment (start 121.9708 95.6742) (end 121.9708 96.5708) (width 0.5) (layer F.Cu) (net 16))
 (segment (start 122.6058 97.2058) (end 125.7198 97.2058) (width 0.5) (layer F.Cu) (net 16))
 (segment (start 121.9708 96.5708) (end 122.6058 97.2058) (width 0.5) (layer F.Cu) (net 16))
 (segment (start 118.237 92.0242) (end 118.237 92.9894) (width 0.5) (layer F.Cu) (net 16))
 (segment (start 118.237 92.9894) (end 119.3546 94.107) (width 0.5) (layer F.Cu) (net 16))
 (segment (start 119.3546 94.107) (end 121.2342 94.107) (width 0.5) (layer F.Cu) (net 16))
 (segment (start 121.2342 94.107) (end 121.9708 94.8436) (width 0.5) (layer F.Cu) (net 16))
 (segment (start 121.9708 94.8436) (end 121.9708 95.6742) (width 0.5) (layer F.Cu) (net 16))
 (segment (start 123.2408 94.6912) (end 123.2408 95.6742) (width 0.5) (layer F.Cu) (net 15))
 (segment (start 120.777 92.2274) (end 123.2408 94.6912) (width 0.5) (layer F.Cu) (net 15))
 (segment (start 120.777 92.0242) (end 120.777 92.2274) (width 0.5) (layer F.Cu) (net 15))
 (segment (start 123.6726 95.123) (end 123.2408 94.6912) (width 0.5) (layer F.Cu) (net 15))
 (segment (start 125.7198 95.123) (end 123.6726 95.123) (width 0.5) (layer F.Cu) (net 15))
 (segment (start 125.7198 95.123) (end 123.6726 95.123) (width 0.5) (layer F.Cu) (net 15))
 (segment (start 123.6726 95.123) (end 123.2408 94.6912) (width 0.5) (layer F.Cu) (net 15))
 (segment (start 120.777 92.0242) (end 120.777 92.2274) (width 0.5) (layer F.Cu) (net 15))
 (segment (start 120.777 92.2274) (end 123.2408 94.6912) (width 0.5) (layer F.Cu) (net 15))
 (segment (start 123.2408 94.6912) (end 123.2408 95.6742) (width 0.5) (layer F.Cu) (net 15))
 (segment (start 121.158 103.9374) (end 121.031 104.0644) (width 0.5) (layer F.Cu) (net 31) (status 30))
 (segment (start 120.7008 102.362) (end 121.031 102.6922) (width 0.5) (layer F.Cu) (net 31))
 (segment (start 121.031 102.6922) (end 121.031 104.0644) (width 0.5) (layer F.Cu) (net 31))
 (segment (start 120.7008 101.0742) (end 120.7008 102.362) (width 0.5) (layer F.Cu) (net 31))
 (segment (start 120.7008 101.0742) (end 120.7008 102.362) (width 0.5) (layer F.Cu) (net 31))
 (segment (start 121.031 102.6922) (end 121.031 104.0644) (width 0.5) (layer F.Cu) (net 31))
 (segment (start 120.7008 102.362) (end 121.031 102.6922) (width 0.5) (layer F.Cu) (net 31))
 (segment (start 121.158 103.9374) (end 121.031 104.0644) (width 0.5) (layer F.Cu) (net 31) (status 30))
 (segment (start 121.9708 99.8728) (end 121.9708 101.0742) (width 0.4) (layer F.Cu) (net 30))
 (segment (start 122.2502 99.5934) (end 121.9708 99.8728) (width 0.4) (layer F.Cu) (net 30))
 (segment (start 123.7234 99.5934) (end 122.2502 99.5934) (width 0.4) (layer F.Cu) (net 30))
 (segment (start 124.7394 100.6094) (end 123.7234 99.5934) (width 0.4) (layer F.Cu) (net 30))
 (segment (start 124.7394 101.0666) (end 124.7394 100.6094) (width 0.4) (layer F.Cu) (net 30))
 (segment (start 125.603 101.9302) (end 124.7394 101.0666) (width 0.4) (layer F.Cu) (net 30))
 (segment (start 126.6698 101.9302) (end 125.603 101.9302) (width 0.4) (layer F.Cu) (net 30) (status 10))
 (segment (start 126.6698 101.9302) (end 125.603 101.9302) (width 0.4) (layer F.Cu) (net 30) (status 10))
 (segment (start 125.603 101.9302) (end 124.7394 101.0666) (width 0.4) (layer F.Cu) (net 30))
 (segment (start 124.7394 101.0666) (end 124.7394 100.6094) (width 0.4) (layer F.Cu) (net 30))
 (segment (start 124.7394 100.6094) (end 123.7234 99.5934) (width 0.4) (layer F.Cu) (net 30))
 (segment (start 123.7234 99.5934) (end 122.2502 99.5934) (width 0.4) (layer F.Cu) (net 30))
 (segment (start 122.2502 99.5934) (end 121.9708 99.8728) (width 0.4) (layer F.Cu) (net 30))
 (segment (start 121.9708 99.8728) (end 121.9708 101.0742) (width 0.4) (layer F.Cu) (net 30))
 (segment (start 120.7008 96.8248) (end 120.7008 95.6742) (width 0.4) (layer F.Cu) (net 28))
 (segment (start 121.9962 98.1202) (end 120.7008 96.8248) (width 0.4) (layer F.Cu) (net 28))
 (segment (start 124.4854 98.1202) (end 121.9962 98.1202) (width 0.4) (layer F.Cu) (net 28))
 (segment (start 125.7554 99.3902) (end 124.4854 98.1202) (width 0.4) (layer F.Cu) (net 28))
 (segment (start 126.6698 99.3902) (end 125.7554 99.3902) (width 0.4) (layer F.Cu) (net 28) (status 10))
 (segment (start 126.6698 99.3902) (end 125.7554 99.3902) (width 0.4) (layer F.Cu) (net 28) (status 10))
 (segment (start 125.7554 99.3902) (end 124.4854 98.1202) (width 0.4) (layer F.Cu) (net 28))
 (segment (start 124.4854 98.1202) (end 121.9962 98.1202) (width 0.4) (layer F.Cu) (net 28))
 (segment (start 121.9962 98.1202) (end 120.7008 96.8248) (width 0.4) (layer F.Cu) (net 28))
 (segment (start 120.7008 96.8248) (end 120.7008 95.6742) (width 0.4) (layer F.Cu) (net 28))
 (segment (start 130.5306 114.9858) (end 133.477 114.9858) (width 0.5) (layer F.Cu) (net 9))
 (segment (start 130.5306 114.9858) (end 133.477 114.9858) (width 0.5) (layer F.Cu) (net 9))
 (segment (start 130.5306 112.4458) (end 133.477 112.4458) (width 0.5) (layer F.Cu) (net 8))
 (segment (start 130.5306 112.4458) (end 133.477 112.4458) (width 0.5) (layer F.Cu) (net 8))
 (segment (start 116.8146 103.2002) (end 113.3602 99.7458) (width 0.5) (layer F.Cu) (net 21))
 (segment (start 113.3602 99.7458) (end 113.157 99.7458) (width 0.5) (layer F.Cu) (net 21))
 (segment (start 116.8146 103.8098) (end 116.8146 103.2002) (width 0.5) (layer F.Cu) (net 21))
 (segment (start 116.8146 103.8098) (end 116.8146 103.2002) (width 0.5) (layer F.Cu) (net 21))
 (segment (start 113.3602 99.7458) (end 113.157 99.7458) (width 0.5) (layer F.Cu) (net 21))
 (segment (start 116.8146 103.2002) (end 113.3602 99.7458) (width 0.5) (layer F.Cu) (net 21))
 (segment (start 115.261 103.555) (end 116.181 103.555) (width 0.5) (layer B.Cu) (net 22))
 (segment (start 113.991 102.285) (end 115.261 103.555) (width 0.5) (layer F.Cu) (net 22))
 (via (at 115.261 103.555) (size 1) (drill 0.5) (layers F.Cu B.Cu) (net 22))
 (via (at 118.401 105.775) (size 1) (drill 0.5) (layers F.Cu B.Cu) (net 22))
 (segment (start 117.8462 106.3498) (end 118.401 105.775) (width 0.5) (layer F.Cu) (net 22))
 (segment (start 117.8462 106.3498) (end 116.8146 106.3498) (width 0.5) (layer F.Cu) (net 22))
 (segment (start 116.181 103.555) (end 118.401 105.775) (width 0.5) (layer B.Cu) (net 22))
 (segment (start 113.991 102.285) (end 113.161 102.285) (width 0.5) (layer F.Cu) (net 22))
 (segment (start 115.2646 105.0798) (end 115.2646 107.9514) (width 0.5) (layer F.Cu) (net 25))
 (segment (start 114.791 109.315) (end 114.201 109.905) (width 0.5) (layer F.Cu) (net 25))
 (segment (start 114.791 108.425) (end 114.791 109.315) (width 0.5) (layer F.Cu) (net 25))
 (segment (start 115.2646 107.9514) (end 114.791 108.425) (width 0.5) (layer F.Cu) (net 25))
 (segment (start 114.201 109.905) (end 113.161 109.905) (width 0.5) (layer F.Cu) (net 25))
 (segment (start 118.3386 103.4034) (end 118.3386 104.4702) (width 0.4) (layer F.Cu) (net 29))
 (segment (start 118.3386 104.4702) (end 117.729 105.0798) (width 0.4) (layer F.Cu) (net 29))
 (segment (start 117.729 105.0798) (end 116.8146 105.0798) (width 0.4) (layer F.Cu) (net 29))
 (segment (start 117.729 105.0798) (end 116.8146 105.0798) (width 0.4) (layer F.Cu) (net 29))
 (segment (start 118.3386 104.4702) (end 117.729 105.0798) (width 0.4) (layer F.Cu) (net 29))
 (segment (start 118.3386 103.4034) (end 118.3386 104.4702) (width 0.4) (layer F.Cu) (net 29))
 (segment (start 125.968198 100.6602) (end 124.190198 98.8822) (width 0.4) (layer F.Cu) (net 29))
 (segment (start 124.190198 98.8822) (end 120.3198 98.8822) (width 0.4) (layer F.Cu) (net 29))
 (segment (start 120.3198 98.8822) (end 119.4562 98.0186) (width 0.4) (layer F.Cu) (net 29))
 (segment (start 119.4562 98.0186) (end 115.697 98.0186) (width 0.4) (layer F.Cu) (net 29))
 (segment (start 115.697 98.0186) (end 115.1382 98.5774) (width 0.4) (layer F.Cu) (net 29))
 (segment (start 115.1382 98.5774) (end 115.1382 100.203) (width 0.4) (layer F.Cu) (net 29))
 (segment (start 115.1382 100.203) (end 118.3386 103.4034) (width 0.4) (layer F.Cu) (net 29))
 (segment (start 126.6698 100.6602) (end 125.968198 100.6602) (width 0.4) (layer F.Cu) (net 29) (status 10))
 (segment (start 126.6698 100.6602) (end 128.905 100.6602) (width 0.5) (layer F.Cu) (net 29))
 (segment (start 128.905 100.6602) (end 128.9558 100.6602) (width 0.5) (layer F.Cu) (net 29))
 (segment (start 128.9558 100.6602) (end 130.0226 99.5934) (width 0.5) (layer F.Cu) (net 29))
 (segment (start 130.0226 99.5934) (end 130.0226 97.089) (width 0.5) (layer F.Cu) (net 29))
 (segment (start 130.0226 99.5934) (end 130.0226 97.089) (width 0.5) (layer F.Cu) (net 29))
 (segment (start 128.9558 100.6602) (end 130.0226 99.5934) (width 0.5) (layer F.Cu) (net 29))
 (segment (start 128.905 100.6602) (end 128.9558 100.6602) (width 0.5) (layer F.Cu) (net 29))
 (segment (start 126.6698 100.6602) (end 128.905 100.6602) (width 0.5) (layer F.Cu) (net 29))
 (segment (start 126.6698 100.6602) (end 125.968198 100.6602) (width 0.4) (layer F.Cu) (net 29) (status 10))
 (segment (start 115.1382 100.203) (end 118.3386 103.4034) (width 0.4) (layer F.Cu) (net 29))
 (segment (start 115.1382 98.5774) (end 115.1382 100.203) (width 0.4) (layer F.Cu) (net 29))
 (segment (start 115.697 98.0186) (end 115.1382 98.5774) (width 0.4) (layer F.Cu) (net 29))
 (segment (start 119.4562 98.0186) (end 115.697 98.0186) (width 0.4) (layer F.Cu) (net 29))
 (segment (start 120.3198 98.8822) (end 119.4562 98.0186) (width 0.4) (layer F.Cu) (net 29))
 (segment (start 124.190198 98.8822) (end 120.3198 98.8822) (width 0.4) (layer F.Cu) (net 29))
 (segment (start 125.968198 100.6602) (end 124.190198 98.8822) (width 0.4) (layer F.Cu) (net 29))
 (segment (start 129.5318 105.819) (end 129.8194 105.819) (width 0.5) (layer F.Cu) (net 33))
 (segment (start 129.8194 104.0486) (end 129.8194 105.819) (width 0.5) (layer F.Cu) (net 33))
 (segment (start 129.8194 104.0486) (end 129.8194 105.819) (width 0.5) (layer F.Cu) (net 33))
 (segment (start 129.5318 105.819) (end 129.8194 105.819) (width 0.5) (layer F.Cu) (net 33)))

